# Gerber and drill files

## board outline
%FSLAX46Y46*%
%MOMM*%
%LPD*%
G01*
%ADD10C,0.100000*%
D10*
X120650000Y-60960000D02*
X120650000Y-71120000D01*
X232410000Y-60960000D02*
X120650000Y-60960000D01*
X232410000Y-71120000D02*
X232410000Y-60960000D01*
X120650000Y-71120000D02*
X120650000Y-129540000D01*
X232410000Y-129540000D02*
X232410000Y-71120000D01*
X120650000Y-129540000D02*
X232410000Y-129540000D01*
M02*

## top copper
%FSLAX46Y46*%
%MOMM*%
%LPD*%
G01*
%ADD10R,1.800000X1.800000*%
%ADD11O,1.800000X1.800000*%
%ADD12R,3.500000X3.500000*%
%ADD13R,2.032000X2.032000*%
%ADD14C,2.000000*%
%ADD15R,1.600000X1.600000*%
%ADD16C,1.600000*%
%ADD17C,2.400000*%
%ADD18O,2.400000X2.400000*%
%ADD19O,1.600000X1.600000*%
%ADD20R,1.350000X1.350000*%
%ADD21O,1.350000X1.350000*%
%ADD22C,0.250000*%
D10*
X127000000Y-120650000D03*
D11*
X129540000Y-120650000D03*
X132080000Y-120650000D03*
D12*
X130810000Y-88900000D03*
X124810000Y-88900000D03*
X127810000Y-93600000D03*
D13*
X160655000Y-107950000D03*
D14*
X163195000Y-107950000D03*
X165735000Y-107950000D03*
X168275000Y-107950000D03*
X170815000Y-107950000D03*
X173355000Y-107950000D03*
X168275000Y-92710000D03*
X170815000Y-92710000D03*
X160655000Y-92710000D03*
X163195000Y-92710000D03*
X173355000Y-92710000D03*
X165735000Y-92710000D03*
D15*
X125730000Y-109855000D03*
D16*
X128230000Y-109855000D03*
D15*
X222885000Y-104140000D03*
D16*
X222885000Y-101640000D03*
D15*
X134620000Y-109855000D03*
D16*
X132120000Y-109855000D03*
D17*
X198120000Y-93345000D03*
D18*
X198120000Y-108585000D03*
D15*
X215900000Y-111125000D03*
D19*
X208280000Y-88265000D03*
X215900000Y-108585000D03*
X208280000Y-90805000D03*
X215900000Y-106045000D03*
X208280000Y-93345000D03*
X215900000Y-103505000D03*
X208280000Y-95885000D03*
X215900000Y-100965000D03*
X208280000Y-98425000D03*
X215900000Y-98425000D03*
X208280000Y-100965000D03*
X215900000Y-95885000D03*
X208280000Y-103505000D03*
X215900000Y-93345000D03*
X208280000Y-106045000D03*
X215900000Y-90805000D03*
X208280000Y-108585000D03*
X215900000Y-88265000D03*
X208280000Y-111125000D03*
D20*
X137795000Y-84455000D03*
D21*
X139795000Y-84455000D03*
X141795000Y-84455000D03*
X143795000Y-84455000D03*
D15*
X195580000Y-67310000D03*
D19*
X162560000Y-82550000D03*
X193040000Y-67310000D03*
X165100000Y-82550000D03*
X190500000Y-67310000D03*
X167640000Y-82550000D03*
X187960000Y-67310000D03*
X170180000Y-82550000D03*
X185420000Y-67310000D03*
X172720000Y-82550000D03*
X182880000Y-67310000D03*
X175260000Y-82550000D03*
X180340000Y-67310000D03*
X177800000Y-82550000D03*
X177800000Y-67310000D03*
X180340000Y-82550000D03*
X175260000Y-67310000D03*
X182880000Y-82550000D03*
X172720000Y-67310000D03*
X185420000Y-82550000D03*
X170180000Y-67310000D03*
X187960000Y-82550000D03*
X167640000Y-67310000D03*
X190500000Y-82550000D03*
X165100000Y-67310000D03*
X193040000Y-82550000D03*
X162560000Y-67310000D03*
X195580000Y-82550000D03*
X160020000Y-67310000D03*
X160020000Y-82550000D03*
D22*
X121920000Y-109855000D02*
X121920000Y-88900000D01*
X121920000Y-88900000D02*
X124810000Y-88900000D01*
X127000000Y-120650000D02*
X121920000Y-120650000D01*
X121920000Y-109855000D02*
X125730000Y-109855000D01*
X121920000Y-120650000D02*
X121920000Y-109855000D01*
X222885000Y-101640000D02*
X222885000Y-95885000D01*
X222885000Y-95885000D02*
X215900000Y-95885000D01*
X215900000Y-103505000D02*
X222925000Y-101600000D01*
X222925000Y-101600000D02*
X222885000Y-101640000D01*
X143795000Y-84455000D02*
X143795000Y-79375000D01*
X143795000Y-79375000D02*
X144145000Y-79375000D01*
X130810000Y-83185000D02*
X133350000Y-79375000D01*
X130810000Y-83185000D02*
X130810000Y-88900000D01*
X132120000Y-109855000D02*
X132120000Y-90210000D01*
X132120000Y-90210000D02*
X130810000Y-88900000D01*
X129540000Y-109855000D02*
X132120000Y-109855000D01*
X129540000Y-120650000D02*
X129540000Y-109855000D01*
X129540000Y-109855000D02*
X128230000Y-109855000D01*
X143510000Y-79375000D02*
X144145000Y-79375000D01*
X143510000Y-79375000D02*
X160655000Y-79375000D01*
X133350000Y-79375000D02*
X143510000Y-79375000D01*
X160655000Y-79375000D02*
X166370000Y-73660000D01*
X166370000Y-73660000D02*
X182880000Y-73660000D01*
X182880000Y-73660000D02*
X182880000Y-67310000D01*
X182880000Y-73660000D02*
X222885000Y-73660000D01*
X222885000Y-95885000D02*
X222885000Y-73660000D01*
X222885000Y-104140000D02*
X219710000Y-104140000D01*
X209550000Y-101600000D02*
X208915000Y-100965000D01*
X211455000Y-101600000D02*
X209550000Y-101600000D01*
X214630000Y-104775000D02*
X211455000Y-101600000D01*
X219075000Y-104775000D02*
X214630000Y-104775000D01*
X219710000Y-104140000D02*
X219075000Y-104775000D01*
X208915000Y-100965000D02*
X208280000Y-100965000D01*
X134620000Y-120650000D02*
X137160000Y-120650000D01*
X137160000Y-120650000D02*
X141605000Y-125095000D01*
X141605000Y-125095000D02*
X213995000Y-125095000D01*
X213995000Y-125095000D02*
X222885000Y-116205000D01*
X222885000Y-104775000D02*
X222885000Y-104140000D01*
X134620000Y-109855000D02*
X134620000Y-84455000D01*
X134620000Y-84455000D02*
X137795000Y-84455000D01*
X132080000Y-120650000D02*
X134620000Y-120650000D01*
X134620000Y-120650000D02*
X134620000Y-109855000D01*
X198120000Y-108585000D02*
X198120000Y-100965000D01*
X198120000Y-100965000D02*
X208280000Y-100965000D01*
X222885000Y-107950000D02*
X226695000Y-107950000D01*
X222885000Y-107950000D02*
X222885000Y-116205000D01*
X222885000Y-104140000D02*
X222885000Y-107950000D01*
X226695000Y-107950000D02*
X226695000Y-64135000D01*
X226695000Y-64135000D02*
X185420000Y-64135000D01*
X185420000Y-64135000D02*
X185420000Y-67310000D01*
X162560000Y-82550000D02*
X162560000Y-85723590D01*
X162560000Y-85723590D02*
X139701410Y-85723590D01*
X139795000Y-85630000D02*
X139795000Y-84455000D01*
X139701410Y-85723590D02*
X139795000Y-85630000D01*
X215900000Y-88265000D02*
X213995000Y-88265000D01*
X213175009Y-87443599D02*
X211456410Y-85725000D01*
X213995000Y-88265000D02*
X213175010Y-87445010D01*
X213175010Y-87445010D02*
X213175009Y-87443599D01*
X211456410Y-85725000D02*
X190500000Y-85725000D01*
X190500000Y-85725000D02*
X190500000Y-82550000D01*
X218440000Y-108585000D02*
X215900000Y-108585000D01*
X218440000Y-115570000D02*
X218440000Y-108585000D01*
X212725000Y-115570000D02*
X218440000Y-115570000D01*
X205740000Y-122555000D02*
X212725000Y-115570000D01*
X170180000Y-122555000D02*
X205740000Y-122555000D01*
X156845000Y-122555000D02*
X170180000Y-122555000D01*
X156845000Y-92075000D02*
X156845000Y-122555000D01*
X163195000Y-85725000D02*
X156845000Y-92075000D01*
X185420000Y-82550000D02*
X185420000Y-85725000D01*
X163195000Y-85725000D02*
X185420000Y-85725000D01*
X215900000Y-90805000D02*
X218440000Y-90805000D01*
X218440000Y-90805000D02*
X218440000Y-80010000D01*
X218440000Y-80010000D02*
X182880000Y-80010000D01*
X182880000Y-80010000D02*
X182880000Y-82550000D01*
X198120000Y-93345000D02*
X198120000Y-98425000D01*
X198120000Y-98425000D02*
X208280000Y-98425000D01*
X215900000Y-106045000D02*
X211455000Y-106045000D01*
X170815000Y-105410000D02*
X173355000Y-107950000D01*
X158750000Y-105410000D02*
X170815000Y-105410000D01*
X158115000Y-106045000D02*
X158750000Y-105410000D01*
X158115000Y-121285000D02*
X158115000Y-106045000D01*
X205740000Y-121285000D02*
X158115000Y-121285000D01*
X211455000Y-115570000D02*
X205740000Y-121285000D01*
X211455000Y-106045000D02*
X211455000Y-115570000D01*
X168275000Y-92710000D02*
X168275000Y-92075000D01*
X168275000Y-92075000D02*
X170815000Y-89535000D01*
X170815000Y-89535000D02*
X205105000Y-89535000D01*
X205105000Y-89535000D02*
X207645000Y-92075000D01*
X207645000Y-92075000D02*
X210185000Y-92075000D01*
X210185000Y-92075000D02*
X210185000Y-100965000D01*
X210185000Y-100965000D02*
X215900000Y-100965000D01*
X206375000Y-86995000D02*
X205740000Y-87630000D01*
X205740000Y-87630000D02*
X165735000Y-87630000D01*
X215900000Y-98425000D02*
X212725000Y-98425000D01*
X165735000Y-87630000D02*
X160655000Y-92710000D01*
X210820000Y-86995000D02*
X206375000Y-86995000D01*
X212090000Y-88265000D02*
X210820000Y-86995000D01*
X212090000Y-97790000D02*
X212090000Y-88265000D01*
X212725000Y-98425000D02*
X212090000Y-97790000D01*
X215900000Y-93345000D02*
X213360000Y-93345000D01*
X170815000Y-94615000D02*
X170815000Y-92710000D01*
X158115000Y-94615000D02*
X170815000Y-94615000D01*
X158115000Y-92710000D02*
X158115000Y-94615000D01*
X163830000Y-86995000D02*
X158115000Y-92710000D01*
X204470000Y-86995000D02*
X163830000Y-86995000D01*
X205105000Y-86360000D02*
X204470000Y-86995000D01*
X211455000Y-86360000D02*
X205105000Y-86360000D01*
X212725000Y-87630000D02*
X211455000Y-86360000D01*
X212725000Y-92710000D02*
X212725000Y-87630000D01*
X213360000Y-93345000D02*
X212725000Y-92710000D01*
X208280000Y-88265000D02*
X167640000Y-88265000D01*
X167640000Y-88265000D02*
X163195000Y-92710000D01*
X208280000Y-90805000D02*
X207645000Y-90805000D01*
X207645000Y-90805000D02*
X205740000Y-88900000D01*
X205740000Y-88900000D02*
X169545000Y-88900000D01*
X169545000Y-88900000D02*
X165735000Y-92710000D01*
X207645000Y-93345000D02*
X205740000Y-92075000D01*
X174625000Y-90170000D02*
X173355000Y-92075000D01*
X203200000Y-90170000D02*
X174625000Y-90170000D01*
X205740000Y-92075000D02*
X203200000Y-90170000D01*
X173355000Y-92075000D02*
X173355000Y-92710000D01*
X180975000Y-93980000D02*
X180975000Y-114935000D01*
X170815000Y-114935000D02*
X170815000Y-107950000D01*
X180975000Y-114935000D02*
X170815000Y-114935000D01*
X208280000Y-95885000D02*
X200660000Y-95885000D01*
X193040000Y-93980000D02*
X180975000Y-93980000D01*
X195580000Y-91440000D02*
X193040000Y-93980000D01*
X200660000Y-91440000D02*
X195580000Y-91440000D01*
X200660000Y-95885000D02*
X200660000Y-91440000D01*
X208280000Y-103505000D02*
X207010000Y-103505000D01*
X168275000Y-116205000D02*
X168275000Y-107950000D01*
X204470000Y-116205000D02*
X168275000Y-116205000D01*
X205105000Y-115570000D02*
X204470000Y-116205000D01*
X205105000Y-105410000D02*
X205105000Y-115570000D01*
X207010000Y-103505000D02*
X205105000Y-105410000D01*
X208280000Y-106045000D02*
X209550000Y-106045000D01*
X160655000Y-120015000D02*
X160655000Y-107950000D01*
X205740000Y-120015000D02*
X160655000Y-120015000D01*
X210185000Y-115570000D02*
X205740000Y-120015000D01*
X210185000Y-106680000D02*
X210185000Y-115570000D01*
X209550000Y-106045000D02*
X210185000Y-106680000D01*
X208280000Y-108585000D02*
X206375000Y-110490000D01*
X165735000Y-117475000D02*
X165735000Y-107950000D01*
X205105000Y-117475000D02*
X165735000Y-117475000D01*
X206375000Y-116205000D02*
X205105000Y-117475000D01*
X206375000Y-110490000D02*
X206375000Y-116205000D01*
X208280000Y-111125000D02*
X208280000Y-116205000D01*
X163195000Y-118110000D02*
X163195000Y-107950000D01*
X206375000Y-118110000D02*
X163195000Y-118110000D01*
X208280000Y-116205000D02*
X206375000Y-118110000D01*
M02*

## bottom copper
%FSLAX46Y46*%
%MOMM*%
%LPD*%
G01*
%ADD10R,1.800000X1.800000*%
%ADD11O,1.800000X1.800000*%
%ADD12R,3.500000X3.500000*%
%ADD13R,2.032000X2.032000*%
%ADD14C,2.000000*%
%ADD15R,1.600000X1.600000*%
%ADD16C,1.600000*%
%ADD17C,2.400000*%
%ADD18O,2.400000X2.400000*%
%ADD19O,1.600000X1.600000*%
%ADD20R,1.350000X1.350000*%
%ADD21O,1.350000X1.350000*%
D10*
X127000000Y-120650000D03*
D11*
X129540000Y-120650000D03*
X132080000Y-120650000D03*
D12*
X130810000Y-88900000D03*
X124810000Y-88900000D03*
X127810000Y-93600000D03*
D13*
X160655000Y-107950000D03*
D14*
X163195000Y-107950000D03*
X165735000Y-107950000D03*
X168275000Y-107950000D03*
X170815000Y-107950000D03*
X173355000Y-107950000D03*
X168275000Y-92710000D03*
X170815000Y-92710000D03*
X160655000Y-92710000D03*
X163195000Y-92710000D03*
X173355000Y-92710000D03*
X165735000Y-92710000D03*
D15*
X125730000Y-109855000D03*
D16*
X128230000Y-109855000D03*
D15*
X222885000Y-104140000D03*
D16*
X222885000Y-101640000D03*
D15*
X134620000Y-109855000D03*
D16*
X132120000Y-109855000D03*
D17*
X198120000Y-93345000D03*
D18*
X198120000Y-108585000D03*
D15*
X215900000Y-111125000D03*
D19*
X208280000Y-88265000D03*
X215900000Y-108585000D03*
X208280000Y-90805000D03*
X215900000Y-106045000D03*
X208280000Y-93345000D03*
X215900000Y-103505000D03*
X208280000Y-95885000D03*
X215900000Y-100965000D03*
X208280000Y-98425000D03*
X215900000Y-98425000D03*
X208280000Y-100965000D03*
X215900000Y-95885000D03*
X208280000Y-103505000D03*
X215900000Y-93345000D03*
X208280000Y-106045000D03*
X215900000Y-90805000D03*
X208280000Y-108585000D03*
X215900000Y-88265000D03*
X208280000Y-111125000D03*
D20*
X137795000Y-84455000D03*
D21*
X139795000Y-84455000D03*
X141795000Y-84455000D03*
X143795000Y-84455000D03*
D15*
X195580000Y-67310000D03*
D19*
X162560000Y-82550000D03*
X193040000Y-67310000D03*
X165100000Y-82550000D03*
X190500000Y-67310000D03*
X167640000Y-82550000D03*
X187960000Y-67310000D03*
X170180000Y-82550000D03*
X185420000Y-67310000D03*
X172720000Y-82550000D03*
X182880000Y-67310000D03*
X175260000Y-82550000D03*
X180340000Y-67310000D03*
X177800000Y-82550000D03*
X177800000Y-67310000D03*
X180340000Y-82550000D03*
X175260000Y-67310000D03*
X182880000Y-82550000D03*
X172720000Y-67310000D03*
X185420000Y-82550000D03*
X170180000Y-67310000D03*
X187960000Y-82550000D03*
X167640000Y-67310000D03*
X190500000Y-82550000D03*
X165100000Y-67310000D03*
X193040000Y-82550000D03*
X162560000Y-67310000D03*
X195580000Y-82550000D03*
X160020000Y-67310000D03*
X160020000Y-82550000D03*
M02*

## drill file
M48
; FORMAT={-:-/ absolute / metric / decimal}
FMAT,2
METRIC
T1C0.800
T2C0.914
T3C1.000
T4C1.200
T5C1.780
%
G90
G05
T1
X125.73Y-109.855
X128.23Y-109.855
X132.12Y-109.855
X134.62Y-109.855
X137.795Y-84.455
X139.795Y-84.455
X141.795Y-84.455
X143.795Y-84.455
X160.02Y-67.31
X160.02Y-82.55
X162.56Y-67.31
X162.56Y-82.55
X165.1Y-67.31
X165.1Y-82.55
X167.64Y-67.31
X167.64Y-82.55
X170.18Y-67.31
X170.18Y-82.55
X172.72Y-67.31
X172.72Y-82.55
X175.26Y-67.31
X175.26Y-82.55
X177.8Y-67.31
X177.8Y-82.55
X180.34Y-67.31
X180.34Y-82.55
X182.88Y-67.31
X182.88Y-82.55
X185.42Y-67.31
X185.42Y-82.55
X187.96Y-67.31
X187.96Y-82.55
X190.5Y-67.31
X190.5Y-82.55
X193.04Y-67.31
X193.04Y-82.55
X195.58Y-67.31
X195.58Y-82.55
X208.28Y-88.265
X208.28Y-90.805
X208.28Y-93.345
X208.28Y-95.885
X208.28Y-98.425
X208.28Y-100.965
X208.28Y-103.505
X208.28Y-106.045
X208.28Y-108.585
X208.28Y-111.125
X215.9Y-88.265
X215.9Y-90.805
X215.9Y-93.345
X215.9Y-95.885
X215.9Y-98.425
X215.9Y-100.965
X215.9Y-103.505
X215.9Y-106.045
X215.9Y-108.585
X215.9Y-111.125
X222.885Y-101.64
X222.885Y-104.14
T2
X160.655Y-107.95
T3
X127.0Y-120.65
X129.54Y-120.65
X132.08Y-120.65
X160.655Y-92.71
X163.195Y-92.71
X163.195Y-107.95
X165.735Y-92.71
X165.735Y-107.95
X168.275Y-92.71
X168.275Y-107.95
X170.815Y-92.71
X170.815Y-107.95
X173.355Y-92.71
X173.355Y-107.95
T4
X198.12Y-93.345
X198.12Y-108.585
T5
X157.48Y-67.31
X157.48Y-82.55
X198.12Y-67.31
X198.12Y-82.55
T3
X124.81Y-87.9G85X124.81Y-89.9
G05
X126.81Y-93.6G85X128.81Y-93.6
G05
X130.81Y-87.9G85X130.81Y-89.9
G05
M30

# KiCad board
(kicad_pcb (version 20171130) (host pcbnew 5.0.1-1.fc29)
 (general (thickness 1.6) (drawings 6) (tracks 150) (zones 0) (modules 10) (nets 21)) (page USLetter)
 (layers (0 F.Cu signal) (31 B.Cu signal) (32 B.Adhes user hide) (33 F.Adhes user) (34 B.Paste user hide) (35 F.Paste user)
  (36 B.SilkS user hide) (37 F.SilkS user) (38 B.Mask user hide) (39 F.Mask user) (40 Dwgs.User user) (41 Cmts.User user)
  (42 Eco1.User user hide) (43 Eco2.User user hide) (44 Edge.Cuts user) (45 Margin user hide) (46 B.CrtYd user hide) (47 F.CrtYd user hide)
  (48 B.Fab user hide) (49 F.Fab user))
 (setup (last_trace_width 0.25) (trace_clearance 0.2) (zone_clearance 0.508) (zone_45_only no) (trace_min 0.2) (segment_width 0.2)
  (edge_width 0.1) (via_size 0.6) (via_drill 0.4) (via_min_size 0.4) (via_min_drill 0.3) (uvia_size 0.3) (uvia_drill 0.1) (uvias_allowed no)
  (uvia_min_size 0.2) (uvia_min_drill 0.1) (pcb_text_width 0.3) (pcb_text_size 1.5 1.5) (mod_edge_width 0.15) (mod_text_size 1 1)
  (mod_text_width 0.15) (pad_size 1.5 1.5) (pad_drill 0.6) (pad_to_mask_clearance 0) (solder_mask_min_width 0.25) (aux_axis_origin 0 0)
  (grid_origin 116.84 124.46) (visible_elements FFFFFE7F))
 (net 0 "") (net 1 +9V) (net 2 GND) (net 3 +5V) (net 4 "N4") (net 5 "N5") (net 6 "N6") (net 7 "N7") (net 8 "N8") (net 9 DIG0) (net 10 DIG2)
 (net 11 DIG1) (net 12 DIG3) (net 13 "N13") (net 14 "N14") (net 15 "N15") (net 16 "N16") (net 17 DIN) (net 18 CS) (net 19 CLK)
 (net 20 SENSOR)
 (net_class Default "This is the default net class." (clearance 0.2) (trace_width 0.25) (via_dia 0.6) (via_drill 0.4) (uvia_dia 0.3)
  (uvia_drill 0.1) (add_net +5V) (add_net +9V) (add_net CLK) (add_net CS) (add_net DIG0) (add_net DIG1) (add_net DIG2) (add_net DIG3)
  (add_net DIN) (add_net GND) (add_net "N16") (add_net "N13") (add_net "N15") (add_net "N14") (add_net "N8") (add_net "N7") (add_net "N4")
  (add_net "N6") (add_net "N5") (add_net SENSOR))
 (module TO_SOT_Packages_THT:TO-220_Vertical (layer F.Cu) (at 127 120.65)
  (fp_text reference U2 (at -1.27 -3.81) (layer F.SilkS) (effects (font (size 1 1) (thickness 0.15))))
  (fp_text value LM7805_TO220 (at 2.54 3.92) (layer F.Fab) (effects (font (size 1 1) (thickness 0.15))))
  (pad 1 thru_hole rect (at 0 0) (size 1.8 1.8) (drill 1) (layers *.Cu *.Mask) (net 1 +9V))
  (pad 2 thru_hole oval (at 2.54 0) (size 1.8 1.8) (drill 1) (layers *.Cu *.Mask) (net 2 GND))
  (pad 3 thru_hole oval (at 5.08 0) (size 1.8 1.8) (drill 1) (layers *.Cu *.Mask) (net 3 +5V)))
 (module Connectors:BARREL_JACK (layer F.Cu) (at 130.81 88.9)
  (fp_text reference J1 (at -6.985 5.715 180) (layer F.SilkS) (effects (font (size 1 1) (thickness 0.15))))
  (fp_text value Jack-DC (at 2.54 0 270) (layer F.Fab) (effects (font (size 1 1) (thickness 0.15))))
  (pad 1 thru_hole rect (at 0 0) (size 3.5 3.5) (drill oval 1 3) (layers *.Cu *.Mask) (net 2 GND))
  (pad 2 thru_hole rect (at -6 0) (size 3.5 3.5) (drill oval 1 3) (layers *.Cu *.Mask) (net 1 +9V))
  (pad 3 thru_hole rect (at -3 4.7) (size 3.5 3.5) (drill oval 3 1) (layers *.Cu *.Mask)))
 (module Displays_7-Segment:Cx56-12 (layer F.Cu) (at 160.655 107.95)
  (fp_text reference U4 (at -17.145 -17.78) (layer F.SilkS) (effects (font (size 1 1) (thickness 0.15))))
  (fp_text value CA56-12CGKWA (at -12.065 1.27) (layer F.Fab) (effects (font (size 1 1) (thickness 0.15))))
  (pad 1 thru_hole rect (at 0 0) (size 2.032 2.032) (drill 0.9144) (layers *.Cu *.Mask) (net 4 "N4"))
  (pad 2 thru_hole circle (at 2.54 0) (size 2 2) (drill 1) (layers *.Cu *.Mask) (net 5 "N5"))
  (pad 3 thru_hole circle (at 5.08 0) (size 2 2) (drill 1) (layers *.Cu *.Mask) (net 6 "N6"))
  (pad 4 thru_hole circle (at 7.62 0) (size 2 2) (drill 1) (layers *.Cu *.Mask) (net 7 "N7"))
  (pad 5 thru_hole circle (at 10.16 0) (size 2 2) (drill 1) (layers *.Cu *.Mask) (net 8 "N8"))
  (pad 6 thru_hole circle (at 12.7 0) (size 2 2) (drill 1) (layers *.Cu *.Mask) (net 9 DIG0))
  (pad 9 thru_hole circle (at 7.62 -15.24) (size 2 2) (drill 1) (layers *.Cu *.Mask) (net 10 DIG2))
  (pad 8 thru_hole circle (at 10.16 -15.24) (size 2 2) (drill 1) (layers *.Cu *.Mask) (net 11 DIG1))
  (pad 12 thru_hole circle (at 0 -15.24) (size 2 2) (drill 1) (layers *.Cu *.Mask) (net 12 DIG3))
  (pad 11 thru_hole circle (at 2.54 -15.24) (size 2 2) (drill 1) (layers *.Cu *.Mask) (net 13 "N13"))
  (pad 7 thru_hole circle (at 12.7 -15.24) (size 2 2) (drill 1) (layers *.Cu *.Mask) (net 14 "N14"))
  (pad 10 thru_hole circle (at 5.08 -15.24) (size 2 2) (drill 1) (layers *.Cu *.Mask) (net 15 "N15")))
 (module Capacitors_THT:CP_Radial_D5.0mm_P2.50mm (layer F.Cu) (at 125.73 109.855)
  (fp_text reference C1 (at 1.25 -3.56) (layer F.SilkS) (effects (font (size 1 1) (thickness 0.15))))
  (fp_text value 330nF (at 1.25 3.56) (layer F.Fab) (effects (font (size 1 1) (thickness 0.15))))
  (pad 1 thru_hole rect (at 0 0) (size 1.6 1.6) (drill 0.8) (layers *.Cu *.Mask) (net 1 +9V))
  (pad 2 thru_hole circle (at 2.5 0) (size 1.6 1.6) (drill 0.8) (layers *.Cu *.Mask) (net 2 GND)))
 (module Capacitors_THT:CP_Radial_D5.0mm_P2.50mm (layer F.Cu) (at 222.885 104.14 90)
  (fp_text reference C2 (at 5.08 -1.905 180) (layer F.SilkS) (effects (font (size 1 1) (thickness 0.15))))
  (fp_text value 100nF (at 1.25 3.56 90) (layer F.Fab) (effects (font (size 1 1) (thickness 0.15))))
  (pad 1 thru_hole rect (at 0 0 90) (size 1.6 1.6) (drill 0.8) (layers *.Cu *.Mask) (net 3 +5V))
  (pad 2 thru_hole circle (at 2.5 0 90) (size 1.6 1.6) (drill 0.8) (layers *.Cu *.Mask) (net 2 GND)))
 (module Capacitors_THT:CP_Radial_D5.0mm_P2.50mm (layer F.Cu) (at 134.62 109.855 180)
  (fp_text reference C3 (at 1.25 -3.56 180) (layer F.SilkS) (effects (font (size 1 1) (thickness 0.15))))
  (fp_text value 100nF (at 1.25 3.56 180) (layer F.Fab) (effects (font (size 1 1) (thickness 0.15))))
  (pad 1 thru_hole rect (at 0 0 180) (size 1.6 1.6) (drill 0.8) (layers *.Cu *.Mask) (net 3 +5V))
  (pad 2 thru_hole circle (at 2.5 0 180) (size 1.6 1.6) (drill 0.8) (layers *.Cu *.Mask) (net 2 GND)))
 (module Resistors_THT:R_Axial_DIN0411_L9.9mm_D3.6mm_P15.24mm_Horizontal (layer F.Cu) (at 198.12 93.345 270)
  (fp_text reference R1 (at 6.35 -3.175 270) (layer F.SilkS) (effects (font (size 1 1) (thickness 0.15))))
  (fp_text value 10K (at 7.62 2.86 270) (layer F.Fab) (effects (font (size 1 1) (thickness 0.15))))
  (pad 1 thru_hole circle (at 0 0 270) (size 2.4 2.4) (drill 1.2) (layers *.Cu *.Mask) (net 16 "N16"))
  (pad 2 thru_hole oval (at 15.24 0 270) (size 2.4 2.4) (drill 1.2) (layers *.Cu *.Mask) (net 3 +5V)))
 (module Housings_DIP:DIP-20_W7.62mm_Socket (layer F.Cu) (at 215.9 111.125 180)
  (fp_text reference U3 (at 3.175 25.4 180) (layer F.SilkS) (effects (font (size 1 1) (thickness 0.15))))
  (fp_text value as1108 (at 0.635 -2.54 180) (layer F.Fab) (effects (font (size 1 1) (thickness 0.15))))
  (pad 1 thru_hole rect (at 0 0 180) (size 1.6 1.6) (drill 0.8) (layers *.Cu *.Mask))
  (pad 11 thru_hole oval (at 7.62 22.86 180) (size 1.6 1.6) (drill 0.8) (layers *.Cu *.Mask) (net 13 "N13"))
  (pad 2 thru_hole oval (at 0 2.54 180) (size 1.6 1.6) (drill 0.8) (layers *.Cu *.Mask) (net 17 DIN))
  (pad 12 thru_hole oval (at 7.62 20.32 180) (size 1.6 1.6) (drill 0.8) (layers *.Cu *.Mask) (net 15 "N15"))
  (pad 3 thru_hole oval (at 0 5.08 180) (size 1.6 1.6) (drill 0.8) (layers *.Cu *.Mask) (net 9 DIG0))
  (pad 13 thru_hole oval (at 7.62 17.78 180) (size 1.6 1.6) (drill 0.8) (layers *.Cu *.Mask) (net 14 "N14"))
  (pad 4 thru_hole oval (at 0 7.62 180) (size 1.6 1.6) (drill 0.8) (layers *.Cu *.Mask) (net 2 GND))
  (pad 14 thru_hole oval (at 7.62 15.24 180) (size 1.6 1.6) (drill 0.8) (layers *.Cu *.Mask) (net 8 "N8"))
  (pad 5 thru_hole oval (at 0 10.16 180) (size 1.6 1.6) (drill 0.8) (layers *.Cu *.Mask) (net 10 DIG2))
  (pad 15 thru_hole oval (at 7.62 12.7 180) (size 1.6 1.6) (drill 0.8) (layers *.Cu *.Mask) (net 16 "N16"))
  (pad 6 thru_hole oval (at 0 12.7 180) (size 1.6 1.6) (drill 0.8) (layers *.Cu *.Mask) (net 12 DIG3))
  (pad 16 thru_hole oval (at 7.62 10.16 180) (size 1.6 1.6) (drill 0.8) (layers *.Cu *.Mask) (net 3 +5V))
  (pad 7 thru_hole oval (at 0 15.24 180) (size 1.6 1.6) (drill 0.8) (layers *.Cu *.Mask) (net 2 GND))
  (pad 17 thru_hole oval (at 7.62 7.62 180) (size 1.6 1.6) (drill 0.8) (layers *.Cu *.Mask) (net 7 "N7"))
  (pad 8 thru_hole oval (at 0 17.78 180) (size 1.6 1.6) (drill 0.8) (layers *.Cu *.Mask) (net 11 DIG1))
  (pad 18 thru_hole oval (at 7.62 5.08 180) (size 1.6 1.6) (drill 0.8) (layers *.Cu *.Mask) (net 4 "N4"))
  (pad 9 thru_hole oval (at 0 20.32 180) (size 1.6 1.6) (drill 0.8) (layers *.Cu *.Mask) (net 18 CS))
  (pad 19 thru_hole oval (at 7.62 2.54 180) (size 1.6 1.6) (drill 0.8) (layers *.Cu *.Mask) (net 6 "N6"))
  (pad 10 thru_hole oval (at 0 22.86 180) (size 1.6 1.6) (drill 0.8) (layers *.Cu *.Mask) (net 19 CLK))
  (pad 20 thru_hole oval (at 7.62 0 180) (size 1.6 1.6) (drill 0.8) (layers *.Cu *.Mask) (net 5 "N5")))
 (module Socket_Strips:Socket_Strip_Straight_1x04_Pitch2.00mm (layer F.Cu) (at 137.795 84.455 90)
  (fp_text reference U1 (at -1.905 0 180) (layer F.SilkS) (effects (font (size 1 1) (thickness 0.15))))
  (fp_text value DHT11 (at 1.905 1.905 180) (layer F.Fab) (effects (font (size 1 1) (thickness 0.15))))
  (pad 1 thru_hole rect (at 0 0 90) (size 1.35 1.35) (drill 0.8) (layers *.Cu *.Mask) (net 3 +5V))
  (pad 2 thru_hole oval (at 0 2 90) (size 1.35 1.35) (drill 0.8) (layers *.Cu *.Mask) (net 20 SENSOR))
  (pad 3 thru_hole oval (at 0 4 90) (size 1.35 1.35) (drill 0.8) (layers *.Cu *.Mask))
  (pad 4 thru_hole oval (at 0 6 90) (size 1.35 1.35) (drill 0.8) (layers *.Cu *.Mask) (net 2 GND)))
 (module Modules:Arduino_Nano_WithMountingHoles (layer F.Cu) (at 195.58 67.31 270)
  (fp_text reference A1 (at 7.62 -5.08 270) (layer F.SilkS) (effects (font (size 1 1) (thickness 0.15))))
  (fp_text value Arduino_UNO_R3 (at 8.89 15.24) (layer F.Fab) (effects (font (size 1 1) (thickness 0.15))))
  (pad 1 thru_hole rect (at 0 0 270) (size 1.6 1.6) (drill 0.8) (layers *.Cu *.Mask))
  (pad 17 thru_hole oval (at 15.24 33.02 270) (size 1.6 1.6) (drill 0.8) (layers *.Cu *.Mask) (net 20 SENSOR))
  (pad 2 thru_hole oval (at 0 2.54 270) (size 1.6 1.6) (drill 0.8) (layers *.Cu *.Mask))
  (pad 18 thru_hole oval (at 15.24 30.48 270) (size 1.6 1.6) (drill 0.8) (layers *.Cu *.Mask))
  (pad 3 thru_hole oval (at 0 5.08 270) (size 1.6 1.6) (drill 0.8) (layers *.Cu *.Mask))
  (pad 19 thru_hole oval (at 15.24 27.94 270) (size 1.6 1.6) (drill 0.8) (layers *.Cu *.Mask))
  (pad 4 thru_hole oval (at 0 7.62 270) (size 1.6 1.6) (drill 0.8) (layers *.Cu *.Mask))
  (pad 20 thru_hole oval (at 15.24 25.4 270) (size 1.6 1.6) (drill 0.8) (layers *.Cu *.Mask))
  (pad 5 thru_hole oval (at 0 10.16 270) (size 1.6 1.6) (drill 0.8) (layers *.Cu *.Mask) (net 3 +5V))
  (pad 21 thru_hole oval (at 15.24 22.86 270) (size 1.6 1.6) (drill 0.8) (layers *.Cu *.Mask))
  (pad 6 thru_hole oval (at 0 12.7 270) (size 1.6 1.6) (drill 0.8) (layers *.Cu *.Mask) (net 2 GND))
  (pad 22 thru_hole oval (at 15.24 20.32 270) (size 1.6 1.6) (drill 0.8) (layers *.Cu *.Mask))
  (pad 7 thru_hole oval (at 0 15.24 270) (size 1.6 1.6) (drill 0.8) (layers *.Cu *.Mask))
  (pad 23 thru_hole oval (at 15.24 17.78 270) (size 1.6 1.6) (drill 0.8) (layers *.Cu *.Mask))
  (pad 8 thru_hole oval (at 0 17.78 270) (size 1.6 1.6) (drill 0.8) (layers *.Cu *.Mask))
  (pad 24 thru_hole oval (at 15.24 15.24 270) (size 1.6 1.6) (drill 0.8) (layers *.Cu *.Mask))
  (pad 9 thru_hole oval (at 0 20.32 270) (size 1.6 1.6) (drill 0.8) (layers *.Cu *.Mask))
  (pad 25 thru_hole oval (at 15.24 12.7 270) (size 1.6 1.6) (drill 0.8) (layers *.Cu *.Mask) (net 18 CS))
  (pad 10 thru_hole oval (at 0 22.86 270) (size 1.6 1.6) (drill 0.8) (layers *.Cu *.Mask))
  (pad 26 thru_hole oval (at 15.24 10.16 270) (size 1.6 1.6) (drill 0.8) (layers *.Cu *.Mask) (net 17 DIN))
  (pad 11 thru_hole oval (at 0 25.4 270) (size 1.6 1.6) (drill 0.8) (layers *.Cu *.Mask))
  (pad 27 thru_hole oval (at 15.24 7.62 270) (size 1.6 1.6) (drill 0.8) (layers *.Cu *.Mask))
  (pad 12 thru_hole oval (at 0 27.94 270) (size 1.6 1.6) (drill 0.8) (layers *.Cu *.Mask))
  (pad 28 thru_hole oval (at 15.24 5.08 270) (size 1.6 1.6) (drill 0.8) (layers *.Cu *.Mask) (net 19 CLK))
  (pad 13 thru_hole oval (at 0 30.48 270) (size 1.6 1.6) (drill 0.8) (layers *.Cu *.Mask))
  (pad 29 thru_hole oval (at 15.24 2.54 270) (size 1.6 1.6) (drill 0.8) (layers *.Cu *.Mask))
  (pad 14 thru_hole oval (at 0 33.02 270) (size 1.6 1.6) (drill 0.8) (layers *.Cu *.Mask))
  (pad 30 thru_hole oval (at 15.24 0 270) (size 1.6 1.6) (drill 0.8) (layers *.Cu *.Mask))
  (pad 15 thru_hole oval (at 0 35.56 270) (size 1.6 1.6) (drill 0.8) (layers *.Cu *.Mask))
  (pad 16 thru_hole oval (at 15.24 35.56 270) (size 1.6 1.6) (drill 0.8) (layers *.Cu *.Mask))
  (pad "" np_thru_hole circle (at 0 -2.54 270) (size 1.78 1.78) (drill 1.78) (layers *.Cu *.Mask))
  (pad "" np_thru_hole circle (at 15.24 -2.54 270) (size 1.78 1.78) (drill 1.78) (layers *.Cu *.Mask))
  (pad "" np_thru_hole circle (at 15.24 38.1 270) (size 1.78 1.78) (drill 1.78) (layers *.Cu *.Mask))
  (pad "" np_thru_hole circle (at 0 38.1 270) (size 1.78 1.78) (drill 1.78) (layers *.Cu *.Mask)))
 (gr_line (start 120.65 60.96) (end 120.65 71.12) (layer Edge.Cuts) (width 0.1))
 (gr_line (start 232.41 60.96) (end 120.65 60.96) (layer Edge.Cuts) (width 0.1))
 (gr_line (start 232.41 71.12) (end 232.41 60.96) (layer Edge.Cuts) (width 0.1))
 (gr_line (start 120.65 71.12) (end 120.65 129.54) (angle 90) (layer Edge.Cuts) (width 0.1))
 (gr_line (start 232.41 129.54) (end 232.41 71.12) (angle 90) (layer Edge.Cuts) (width 0.1))
 (gr_line (start 120.65 129.54) (end 232.41 129.54) (angle 90) (layer Edge.Cuts) (width 0.1))
 (segment (start 121.92 109.855) (end 121.92 88.9) (width 0.25) (layer F.Cu) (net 1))
 (segment (start 121.92 88.9) (end 124.81 88.9) (width 0.25) (layer F.Cu) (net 1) (status 20))
 (segment (start 127 120.65) (end 121.92 120.65) (width 0.25) (layer F.Cu) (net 1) (status 10))
 (segment (start 121.92 109.855) (end 125.73 109.855) (width 0.25) (layer F.Cu) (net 1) (status 20))
 (segment (start 121.92 120.65) (end 121.92 109.855) (width 0.25) (layer F.Cu) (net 1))
 (segment (start 222.885 101.64) (end 222.885 95.885) (width 0.25) (layer F.Cu) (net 2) (status 10))
 (segment (start 222.885 95.885) (end 215.9 95.885) (width 0.25) (layer F.Cu) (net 2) (status 20))
 (segment (start 215.9 103.505) (end 222.925 101.6) (width 0.25) (layer F.Cu) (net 2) (status 30))
 (segment (start 222.925 101.6) (end 222.885 101.64) (width 0.25) (layer F.Cu) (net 2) (status 30))
 (segment (start 143.795 84.455) (end 143.795 79.375) (width 0.25) (layer F.Cu) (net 2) (status 10))
 (segment (start 143.795 79.375) (end 144.145 79.375) (width 0.25) (layer F.Cu) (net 2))
 (segment (start 130.81 83.185) (end 133.35 79.375) (width 0.25) (layer F.Cu) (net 2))
 (segment (start 130.81 83.185) (end 130.81 88.9) (width 0.25) (layer F.Cu) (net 2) (status 20))
 (segment (start 132.12 109.855) (end 132.12 90.21) (width 0.25) (layer F.Cu) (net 2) (status 30))
 (segment (start 132.12 90.21) (end 130.81 88.9) (width 0.25) (layer F.Cu) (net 2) (status 30))
 (segment (start 129.54 109.855) (end 132.12 109.855) (width 0.25) (layer F.Cu) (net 2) (status 20))
 (segment (start 129.54 120.65) (end 129.54 109.855) (width 0.25) (layer F.Cu) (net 2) (status 10))
 (segment (start 129.54 109.855) (end 128.23 109.855) (width 0.25) (layer F.Cu) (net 2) (status 20))
 (segment (start 143.51 79.375) (end 144.145 79.375) (width 0.25) (layer F.Cu) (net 2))
 (segment (start 143.51 79.375) (end 160.655 79.375) (width 0.25) (layer F.Cu) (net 2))
 (segment (start 133.35 79.375) (end 143.51 79.375) (width 0.25) (layer F.Cu) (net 2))
 (segment (start 160.655 79.375) (end 166.37 73.66) (width 0.25) (layer F.Cu) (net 2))
 (segment (start 166.37 73.66) (end 182.88 73.66) (width 0.25) (layer F.Cu) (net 2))
 (segment (start 182.88 73.66) (end 182.88 67.31) (width 0.25) (layer F.Cu) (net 2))
 (segment (start 182.88 73.66) (end 222.885 73.66) (width 0.25) (layer F.Cu) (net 2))
 (segment (start 222.885 95.885) (end 222.885 73.66) (width 0.25) (layer F.Cu) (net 2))
 (segment (start 222.885 104.14) (end 219.71 104.14) (width 0.25) (layer F.Cu) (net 3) (status 10))
 (segment (start 209.55 101.6) (end 208.915 100.965) (width 0.25) (layer F.Cu) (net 3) (status 20))
 (segment (start 211.455 101.6) (end 209.55 101.6) (width 0.25) (layer F.Cu) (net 3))
 (segment (start 214.63 104.775) (end 211.455 101.6) (width 0.25) (layer F.Cu) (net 3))
 (segment (start 219.075 104.775) (end 214.63 104.775) (width 0.25) (layer F.Cu) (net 3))
 (segment (start 219.71 104.14) (end 219.075 104.775) (width 0.25) (layer F.Cu) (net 3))
 (segment (start 208.915 100.965) (end 208.28 100.965) (width 0.25) (layer F.Cu) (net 3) (status 30))
 (segment (start 134.62 120.65) (end 137.16 120.65) (width 0.25) (layer F.Cu) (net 3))
 (segment (start 137.16 120.65) (end 141.605 125.095) (width 0.25) (layer F.Cu) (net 3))
 (segment (start 141.605 125.095) (end 213.995 125.095) (width 0.25) (layer F.Cu) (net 3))
 (segment (start 213.995 125.095) (end 222.885 116.205) (width 0.25) (layer F.Cu) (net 3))
 (segment (start 222.885 104.775) (end 222.885 104.14) (width 0.25) (layer F.Cu) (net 3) (status 30))
 (segment (start 134.62 109.855) (end 134.62 84.455) (width 0.25) (layer F.Cu) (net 3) (status 10))
 (segment (start 134.62 84.455) (end 137.795 84.455) (width 0.25) (layer F.Cu) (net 3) (status 20))
 (segment (start 132.08 120.65) (end 134.62 120.65) (width 0.25) (layer F.Cu) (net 3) (status 10))
 (segment (start 134.62 120.65) (end 134.62 109.855) (width 0.25) (layer F.Cu) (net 3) (status 20))
 (segment (start 198.12 108.585) (end 198.12 100.965) (width 0.25) (layer F.Cu) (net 3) (status 10))
 (segment (start 198.12 100.965) (end 208.28 100.965) (width 0.25) (layer F.Cu) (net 3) (status 20))
 (segment (start 222.885 107.95) (end 226.695 107.95) (width 0.25) (layer F.Cu) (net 3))
 (segment (start 222.885 107.95) (end 222.885 116.205) (width 0.25) (layer F.Cu) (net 3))
 (segment (start 222.885 104.14) (end 222.885 107.95) (width 0.25) (layer F.Cu) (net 3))
 (segment (start 226.695 107.95) (end 226.695 64.135) (width 0.25) (layer F.Cu) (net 3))
 (segment (start 226.695 64.135) (end 185.42 64.135) (width 0.25) (layer F.Cu) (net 3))
 (segment (start 185.42 64.135) (end 185.42 67.31) (width 0.25) (layer F.Cu) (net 3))
 (segment (start 162.56 82.55) (end 162.56 85.72359) (width 0.25) (layer F.Cu) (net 20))
 (segment (start 162.56 85.72359) (end 139.70141 85.72359) (width 0.25) (layer F.Cu) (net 20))
 (segment (start 139.795 85.63) (end 139.795 84.455) (width 0.25) (layer F.Cu) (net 20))
 (segment (start 139.70141 85.72359) (end 139.795 85.63) (width 0.25) (layer F.Cu) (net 20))
 (segment (start 215.9 88.265) (end 213.995 88.265) (width 0.25) (layer F.Cu) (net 19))
 (segment (start 213.175009 87.443599) (end 211.45641 85.725) (width 0.25) (layer F.Cu) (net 19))
 (segment (start 213.995 88.265) (end 213.17501 87.44501) (width 0.25) (layer F.Cu) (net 19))
 (segment (start 213.17501 87.44501) (end 213.175009 87.443599) (width 0.25) (layer F.Cu) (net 19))
 (segment (start 211.45641 85.725) (end 190.5 85.725) (width 0.25) (layer F.Cu) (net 19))
 (segment (start 190.5 85.725) (end 190.5 82.55) (width 0.25) (layer F.Cu) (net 19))
 (segment (start 218.44 108.585) (end 215.9 108.585) (width 0.25) (layer F.Cu) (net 17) (status 20))
 (segment (start 218.44 115.57) (end 218.44 108.585) (width 0.25) (layer F.Cu) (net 17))
 (segment (start 212.725 115.57) (end 218.44 115.57) (width 0.25) (layer F.Cu) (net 17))
 (segment (start 205.74 122.555) (end 212.725 115.57) (width 0.25) (layer F.Cu) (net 17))
 (segment (start 170.18 122.555) (end 205.74 122.555) (width 0.25) (layer F.Cu) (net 17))
 (segment (start 156.845 122.555) (end 170.18 122.555) (width 0.25) (layer F.Cu) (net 17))
 (segment (start 156.845 92.075) (end 156.845 122.555) (width 0.25) (layer F.Cu) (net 17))
 (segment (start 163.195 85.725) (end 156.845 92.075) (width 0.25) (layer F.Cu) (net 17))
 (segment (start 185.42 82.55) (end 185.42 85.725) (width 0.25) (layer F.Cu) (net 17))
 (segment (start 163.195 85.725) (end 185.42 85.725) (width 0.25) (layer F.Cu) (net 17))
 (segment (start 215.9 90.805) (end 218.44 90.805) (width 0.25) (layer F.Cu) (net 18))
 (segment (start 218.44 90.805) (end 218.44 80.01) (width 0.25) (layer F.Cu) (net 18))
 (segment (start 218.44 80.01) (end 182.88 80.01) (width 0.25) (layer F.Cu) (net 18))
 (segment (start 182.88 80.01) (end 182.88 82.55) (width 0.25) (layer F.Cu) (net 18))
 (segment (start 198.12 93.345) (end 198.12 98.425) (width 0.25) (layer F.Cu) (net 16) (status 10))
 (segment (start 198.12 98.425) (end 208.28 98.425) (width 0.25) (layer F.Cu) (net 16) (status 20))
 (segment (start 215.9 106.045) (end 211.455 106.045) (width 0.25) (layer F.Cu) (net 9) (status 10))
 (segment (start 170.815 105.41) (end 173.355 107.95) (width 0.25) (layer F.Cu) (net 9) (status 20))
 (segment (start 158.75 105.41) (end 170.815 105.41) (width 0.25) (layer F.Cu) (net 9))
 (segment (start 158.115 106.045) (end 158.75 105.41) (width 0.25) (layer F.Cu) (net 9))
 (segment (start 158.115 121.285) (end 158.115 106.045) (width 0.25) (layer F.Cu) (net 9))
 (segment (start 205.74 121.285) (end 158.115 121.285) (width 0.25) (layer F.Cu) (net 9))
 (segment (start 211.455 115.57) (end 205.74 121.285) (width 0.25) (layer F.Cu) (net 9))
 (segment (start 211.455 106.045) (end 211.455 115.57) (width 0.25) (layer F.Cu) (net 9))
 (segment (start 168.275 92.71) (end 168.275 92.075) (width 0.25) (layer F.Cu) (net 10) (status 30))
 (segment (start 168.275 92.075) (end 170.815 89.535) (width 0.25) (layer F.Cu) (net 10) (status 10))
 (segment (start 170.815 89.535) (end 205.105 89.535) (width 0.25) (layer F.Cu) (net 10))
 (segment (start 205.105 89.535) (end 207.645 92.075) (width 0.25) (layer F.Cu) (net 10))
 (segment (start 207.645 92.075) (end 210.185 92.075) (width 0.25) (layer F.Cu) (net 10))
 (segment (start 210.185 92.075) (end 210.185 100.965) (width 0.25) (layer F.Cu) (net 10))
 (segment (start 210.185 100.965) (end 215.9 100.965) (width 0.25) (layer F.Cu) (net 10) (status 20))
 (segment (start 206.375 86.995) (end 205.74 87.63) (width 0.25) (layer F.Cu) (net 12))
 (segment (start 205.74 87.63) (end 165.735 87.63) (width 0.25) (layer F.Cu) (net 12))
 (segment (start 215.9 98.425) (end 212.725 98.425) (width 0.25) (layer F.Cu) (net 12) (status 10))
 (segment (start 165.735 87.63) (end 160.655 92.71) (width 0.25) (layer F.Cu) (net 12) (status 20))
 (segment (start 210.82 86.995) (end 206.375 86.995) (width 0.25) (layer F.Cu) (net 12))
 (segment (start 212.09 88.265) (end 210.82 86.995) (width 0.25) (layer F.Cu) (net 12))
 (segment (start 212.09 97.79) (end 212.09 88.265) (width 0.25) (layer F.Cu) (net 12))
 (segment (start 212.725 98.425) (end 212.09 97.79) (width 0.25) (layer F.Cu) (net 12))
 (segment (start 215.9 93.345) (end 213.36 93.345) (width 0.25) (layer F.Cu) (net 11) (status 10))
 (segment (start 170.815 94.615) (end 170.815 92.71) (width 0.25) (layer F.Cu) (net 11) (status 20))
 (segment (start 158.115 94.615) (end 170.815 94.615) (width 0.25) (layer F.Cu) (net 11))
 (segment (start 158.115 92.71) (end 158.115 94.615) (width 0.25) (layer F.Cu) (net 11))
 (segment (start 163.83 86.995) (end 158.115 92.71) (width 0.25) (layer F.Cu) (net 11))
 (segment (start 204.47 86.995) (end 163.83 86.995) (width 0.25) (layer F.Cu) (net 11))
 (segment (start 205.105 86.36) (end 204.47 86.995) (width 0.25) (layer F.Cu) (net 11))
 (segment (start 211.455 86.36) (end 205.105 86.36) (width 0.25) (layer F.Cu) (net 11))
 (segment (start 212.725 87.63) (end 211.455 86.36) (width 0.25) (layer F.Cu) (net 11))
 (segment (start 212.725 92.71) (end 212.725 87.63) (width 0.25) (layer F.Cu) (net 11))
 (segment (start 213.36 93.345) (end 212.725 92.71) (width 0.25) (layer F.Cu) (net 11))
 (segment (start 208.28 88.265) (end 167.64 88.265) (width 0.25) (layer F.Cu) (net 13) (status 10))
 (segment (start 167.64 88.265) (end 163.195 92.71) (width 0.25) (layer F.Cu) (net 13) (status 20))
 (segment (start 208.28 90.805) (end 207.645 90.805) (width 0.25) (layer F.Cu) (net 15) (status 30))
 (segment (start 207.645 90.805) (end 205.74 88.9) (width 0.25) (layer F.Cu) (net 15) (status 10))
 (segment (start 205.74 88.9) (end 169.545 88.9) (width 0.25) (layer F.Cu) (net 15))
 (segment (start 169.545 88.9) (end 165.735 92.71) (width 0.25) (layer F.Cu) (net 15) (status 20))
 (segment (start 207.645 93.345) (end 205.74 92.075) (width 0.25) (layer F.Cu) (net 14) (status 10))
 (segment (start 174.625 90.17) (end 173.355 92.075) (width 0.25) (layer F.Cu) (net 14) (status 20))
 (segment (start 203.2 90.17) (end 174.625 90.17) (width 0.25) (layer F.Cu) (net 14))
 (segment (start 205.74 92.075) (end 203.2 90.17) (width 0.25) (layer F.Cu) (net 14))
 (segment (start 173.355 92.075) (end 173.355 92.71) (width 0.25) (layer F.Cu) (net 14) (status 30))
 (segment (start 180.975 93.98) (end 180.975 114.935) (width 0.25) (layer F.Cu) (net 8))
 (segment (start 170.815 114.935) (end 170.815 107.95) (width 0.25) (layer F.Cu) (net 8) (status 20))
 (segment (start 180.975 114.935) (end 170.815 114.935) (width 0.25) (layer F.Cu) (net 8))
 (segment (start 208.28 95.885) (end 200.66 95.885) (width 0.25) (layer F.Cu) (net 8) (status 10))
 (segment (start 193.04 93.98) (end 180.975 93.98) (width 0.25) (layer F.Cu) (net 8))
 (segment (start 195.58 91.44) (end 193.04 93.98) (width 0.25) (layer F.Cu) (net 8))
 (segment (start 200.66 91.44) (end 195.58 91.44) (width 0.25) (layer F.Cu) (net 8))
 (segment (start 200.66 95.885) (end 200.66 91.44) (width 0.25) (layer F.Cu) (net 8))
 (segment (start 208.28 103.505) (end 207.01 103.505) (width 0.25) (layer F.Cu) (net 7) (status 10))
 (segment (start 168.275 116.205) (end 168.275 107.95) (width 0.25) (layer F.Cu) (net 7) (status 20))
 (segment (start 204.47 116.205) (end 168.275 116.205) (width 0.25) (layer F.Cu) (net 7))
 (segment (start 205.105 115.57) (end 204.47 116.205) (width 0.25) (layer F.Cu) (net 7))
 (segment (start 205.105 105.41) (end 205.105 115.57) (width 0.25) (layer F.Cu) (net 7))
 (segment (start 207.01 103.505) (end 205.105 105.41) (width 0.25) (layer F.Cu) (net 7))
 (segment (start 208.28 106.045) (end 209.55 106.045) (width 0.25) (layer F.Cu) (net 4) (status 10))
 (segment (start 160.655 120.015) (end 160.655 107.95) (width 0.25) (layer F.Cu) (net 4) (status 20))
 (segment (start 205.74 120.015) (end 160.655 120.015) (width 0.25) (layer F.Cu) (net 4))
 (segment (start 210.185 115.57) (end 205.74 120.015) (width 0.25) (layer F.Cu) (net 4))
 (segment (start 210.185 106.68) (end 210.185 115.57) (width 0.25) (layer F.Cu) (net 4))
 (segment (start 209.55 106.045) (end 210.185 106.68) (width 0.25) (layer F.Cu) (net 4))
 (segment (start 208.28 108.585) (end 206.375 110.49) (width 0.25) (layer F.Cu) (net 6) (status 10))
 (segment (start 165.735 117.475) (end 165.735 107.95) (width 0.25) (layer F.Cu) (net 6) (status 20))
 (segment (start 205.105 117.475) (end 165.735 117.475) (width 0.25) (layer F.Cu) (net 6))
 (segment (start 206.375 116.205) (end 205.105 117.475) (width 0.25) (layer F.Cu) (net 6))
 (segment (start 206.375 110.49) (end 206.375 116.205) (width 0.25) (layer F.Cu) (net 6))
 (segment (start 208.28 111.125) (end 208.28 116.205) (width 0.25) (layer F.Cu) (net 5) (status 10))
 (segment (start 163.195 118.11) (end 163.195 107.95) (width 0.25) (layer F.Cu) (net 5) (status 20))
 (segment (start 206.375 118.11) (end 163.195 118.11) (width 0.25) (layer F.Cu) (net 5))
 (segment (start 208.28 116.205) (end 206.375 118.11) (width 0.25) (layer F.Cu) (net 5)))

